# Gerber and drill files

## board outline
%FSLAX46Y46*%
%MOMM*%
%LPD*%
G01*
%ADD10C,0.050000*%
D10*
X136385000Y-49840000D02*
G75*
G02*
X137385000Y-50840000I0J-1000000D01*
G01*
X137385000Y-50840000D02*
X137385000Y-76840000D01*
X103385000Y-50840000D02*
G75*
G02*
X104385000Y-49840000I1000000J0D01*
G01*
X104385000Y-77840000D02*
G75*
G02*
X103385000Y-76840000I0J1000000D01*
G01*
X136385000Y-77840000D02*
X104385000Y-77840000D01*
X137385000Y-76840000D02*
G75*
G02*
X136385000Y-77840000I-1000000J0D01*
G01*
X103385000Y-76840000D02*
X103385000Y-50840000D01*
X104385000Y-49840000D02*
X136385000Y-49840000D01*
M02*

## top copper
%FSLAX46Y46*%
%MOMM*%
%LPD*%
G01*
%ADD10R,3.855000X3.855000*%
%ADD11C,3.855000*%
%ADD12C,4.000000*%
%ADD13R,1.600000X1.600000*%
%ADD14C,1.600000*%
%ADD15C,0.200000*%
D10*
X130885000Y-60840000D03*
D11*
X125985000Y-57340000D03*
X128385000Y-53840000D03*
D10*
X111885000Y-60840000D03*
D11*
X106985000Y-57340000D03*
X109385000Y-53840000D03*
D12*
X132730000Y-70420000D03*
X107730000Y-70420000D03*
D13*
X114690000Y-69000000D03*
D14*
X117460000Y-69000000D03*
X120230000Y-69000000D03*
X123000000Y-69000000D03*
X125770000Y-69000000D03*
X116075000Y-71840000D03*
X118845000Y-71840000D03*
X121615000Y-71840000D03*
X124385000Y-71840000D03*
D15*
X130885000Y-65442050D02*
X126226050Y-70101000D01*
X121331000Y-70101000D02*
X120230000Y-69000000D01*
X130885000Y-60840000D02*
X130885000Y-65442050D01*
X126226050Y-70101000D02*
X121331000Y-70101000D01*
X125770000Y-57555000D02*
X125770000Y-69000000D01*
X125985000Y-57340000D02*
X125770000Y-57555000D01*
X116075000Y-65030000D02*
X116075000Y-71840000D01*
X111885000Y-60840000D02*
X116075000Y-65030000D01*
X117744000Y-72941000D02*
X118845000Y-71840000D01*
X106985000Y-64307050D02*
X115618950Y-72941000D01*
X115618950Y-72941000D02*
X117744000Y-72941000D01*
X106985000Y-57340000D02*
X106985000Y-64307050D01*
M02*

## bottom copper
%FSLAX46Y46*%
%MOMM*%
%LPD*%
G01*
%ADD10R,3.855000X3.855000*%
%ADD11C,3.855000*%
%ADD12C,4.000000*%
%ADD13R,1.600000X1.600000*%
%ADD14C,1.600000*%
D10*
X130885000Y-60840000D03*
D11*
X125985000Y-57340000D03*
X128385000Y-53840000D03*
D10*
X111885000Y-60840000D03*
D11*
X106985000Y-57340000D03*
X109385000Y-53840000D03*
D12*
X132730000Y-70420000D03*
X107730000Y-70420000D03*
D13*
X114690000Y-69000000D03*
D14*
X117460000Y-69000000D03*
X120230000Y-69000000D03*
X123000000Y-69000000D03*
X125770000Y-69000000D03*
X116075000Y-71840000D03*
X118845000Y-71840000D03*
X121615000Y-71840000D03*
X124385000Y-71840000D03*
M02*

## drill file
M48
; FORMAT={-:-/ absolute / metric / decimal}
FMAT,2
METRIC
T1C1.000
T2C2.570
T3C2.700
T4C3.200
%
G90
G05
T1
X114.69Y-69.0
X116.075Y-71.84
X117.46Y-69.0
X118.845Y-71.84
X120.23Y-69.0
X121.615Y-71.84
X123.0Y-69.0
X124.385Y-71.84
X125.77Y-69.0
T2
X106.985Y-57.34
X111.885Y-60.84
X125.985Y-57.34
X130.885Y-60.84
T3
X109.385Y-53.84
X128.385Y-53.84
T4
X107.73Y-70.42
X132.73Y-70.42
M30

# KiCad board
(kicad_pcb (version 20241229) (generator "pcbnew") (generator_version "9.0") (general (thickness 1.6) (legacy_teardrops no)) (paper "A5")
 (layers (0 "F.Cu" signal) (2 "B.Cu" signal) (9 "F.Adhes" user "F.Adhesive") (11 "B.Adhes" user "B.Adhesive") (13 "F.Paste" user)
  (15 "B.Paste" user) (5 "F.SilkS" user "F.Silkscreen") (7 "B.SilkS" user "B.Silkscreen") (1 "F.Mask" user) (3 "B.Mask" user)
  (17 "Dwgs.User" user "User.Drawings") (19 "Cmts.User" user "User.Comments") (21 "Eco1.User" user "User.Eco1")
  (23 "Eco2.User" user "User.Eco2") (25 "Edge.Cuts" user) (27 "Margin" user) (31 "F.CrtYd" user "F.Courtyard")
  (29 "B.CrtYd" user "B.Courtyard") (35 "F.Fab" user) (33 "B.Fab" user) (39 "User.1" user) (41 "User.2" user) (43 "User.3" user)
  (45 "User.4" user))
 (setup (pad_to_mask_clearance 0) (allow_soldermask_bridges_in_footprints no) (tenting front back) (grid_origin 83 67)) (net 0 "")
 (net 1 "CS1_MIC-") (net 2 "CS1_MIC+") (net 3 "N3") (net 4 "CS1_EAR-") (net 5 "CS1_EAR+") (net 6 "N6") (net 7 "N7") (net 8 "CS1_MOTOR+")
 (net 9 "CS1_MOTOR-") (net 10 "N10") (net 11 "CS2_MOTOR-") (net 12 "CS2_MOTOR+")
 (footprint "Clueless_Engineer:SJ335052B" (layer "F.Cu") (at 130.885 60.84)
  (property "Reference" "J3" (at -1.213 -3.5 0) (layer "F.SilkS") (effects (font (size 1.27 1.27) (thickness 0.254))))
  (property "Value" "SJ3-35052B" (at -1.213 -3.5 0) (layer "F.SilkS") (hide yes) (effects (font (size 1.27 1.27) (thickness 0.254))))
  (pad "1" thru_hole rect (at 0 0) (size 3.855 3.855) (drill 2.57) (layers "*.Cu" "*.Mask") (remove_unused_layers no) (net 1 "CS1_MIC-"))
  (pad "2" thru_hole circle (at -4.9 -3.5) (size 3.855 3.855) (drill 2.57) (layers "*.Cu" "*.Mask") (remove_unused_layers no)
   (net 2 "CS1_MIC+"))
  (pad "4" thru_hole circle (at -2.5 -7) (size 3.855 3.855) (drill 2.7) (layers "*.Cu" "*.Mask") (remove_unused_layers no) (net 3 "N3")))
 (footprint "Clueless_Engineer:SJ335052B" (layer "F.Cu") (at 111.885 60.84)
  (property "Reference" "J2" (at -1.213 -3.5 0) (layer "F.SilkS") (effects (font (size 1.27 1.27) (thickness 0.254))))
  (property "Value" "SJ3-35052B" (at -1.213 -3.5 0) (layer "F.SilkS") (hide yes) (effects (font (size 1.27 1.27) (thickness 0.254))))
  (pad "1" thru_hole rect (at 0 0) (size 3.855 3.855) (drill 2.57) (layers "*.Cu" "*.Mask") (remove_unused_layers no) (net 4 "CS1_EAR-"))
  (pad "2" thru_hole circle (at -4.9 -3.5) (size 3.855 3.855) (drill 2.57) (layers "*.Cu" "*.Mask") (remove_unused_layers no)
   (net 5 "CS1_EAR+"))
  (pad "4" thru_hole circle (at -2.5 -7) (size 3.855 3.855) (drill 2.7) (layers "*.Cu" "*.Mask") (remove_unused_layers no) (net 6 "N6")))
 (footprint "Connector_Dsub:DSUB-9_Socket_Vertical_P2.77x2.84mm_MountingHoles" (layer "B.Cu") (at 114.69 69 180)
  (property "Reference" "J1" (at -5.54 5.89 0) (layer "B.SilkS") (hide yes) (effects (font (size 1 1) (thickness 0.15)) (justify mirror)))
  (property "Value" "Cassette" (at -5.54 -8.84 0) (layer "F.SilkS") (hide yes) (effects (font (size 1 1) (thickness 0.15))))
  (pad "0" thru_hole circle (at -18.04 -1.42 180) (size 4 4) (drill 3.2) (layers "*.Cu" "*.Mask") (remove_unused_layers no) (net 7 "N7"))
  (pad "0" thru_hole circle (at 6.96 -1.42 180) (size 4 4) (drill 3.2) (layers "*.Cu" "*.Mask") (remove_unused_layers no) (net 7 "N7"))
  (pad "1" thru_hole rect (at 0 0 180) (size 1.6 1.6) (drill 1) (layers "*.Cu" "*.Mask") (remove_unused_layers no) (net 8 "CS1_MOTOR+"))
  (pad "2" thru_hole circle (at -2.77 0 180) (size 1.6 1.6) (drill 1) (layers "*.Cu" "*.Mask") (remove_unused_layers no)
   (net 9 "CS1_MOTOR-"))
  (pad "3" thru_hole circle (at -5.54 0 180) (size 1.6 1.6) (drill 1) (layers "*.Cu" "*.Mask") (remove_unused_layers no) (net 1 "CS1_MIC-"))
  (pad "4" thru_hole circle (at -8.31 0 180) (size 1.6 1.6) (drill 1) (layers "*.Cu" "*.Mask") (remove_unused_layers no) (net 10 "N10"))
  (pad "5" thru_hole circle (at -11.08 0 180) (size 1.6 1.6) (drill 1) (layers "*.Cu" "*.Mask") (remove_unused_layers no) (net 2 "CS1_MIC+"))
  (pad "6" thru_hole circle (at -1.385 -2.84 180) (size 1.6 1.6) (drill 1) (layers "*.Cu" "*.Mask") (remove_unused_layers no)
   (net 4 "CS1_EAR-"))
  (pad "7" thru_hole circle (at -4.155 -2.84 180) (size 1.6 1.6) (drill 1) (layers "*.Cu" "*.Mask") (remove_unused_layers no)
   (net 5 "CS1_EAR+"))
  (pad "8" thru_hole circle (at -6.925 -2.84 180) (size 1.6 1.6) (drill 1) (layers "*.Cu" "*.Mask") (remove_unused_layers no)
   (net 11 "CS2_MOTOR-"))
  (pad "9" thru_hole circle (at -9.695 -2.84 180) (size 1.6 1.6) (drill 1) (layers "*.Cu" "*.Mask") (remove_unused_layers no)
   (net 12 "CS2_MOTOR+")))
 (gr_arc (start 136.385 49.84) (mid 137.092107 50.132893) (end 137.385 50.84) (stroke (width 0.05) (type default)) (layer "Edge.Cuts"))
 (gr_line (start 137.385 50.84) (end 137.385 76.84) (stroke (width 0.05) (type default)) (layer "Edge.Cuts"))
 (gr_arc (start 103.385 50.84) (mid 103.677893 50.132893) (end 104.385 49.84) (stroke (width 0.05) (type default)) (layer "Edge.Cuts"))
 (gr_arc (start 104.385 77.84) (mid 103.677893 77.547107) (end 103.385 76.84) (stroke (width 0.05) (type default)) (layer "Edge.Cuts"))
 (gr_line (start 136.385 77.84) (end 104.385 77.84) (stroke (width 0.05) (type default)) (layer "Edge.Cuts"))
 (gr_arc (start 137.385 76.84) (mid 137.092107 77.547107) (end 136.385 77.84) (stroke (width 0.05) (type default)) (layer "Edge.Cuts"))
 (gr_line (start 103.385 76.84) (end 103.385 50.84) (stroke (width 0.05) (type default)) (layer "Edge.Cuts"))
 (gr_line (start 104.385 49.84) (end 136.385 49.84) (stroke (width 0.05) (type default)) (layer "Edge.Cuts"))
 (segment (start 130.885 65.44205) (end 126.22605 70.101) (width 0.2) (layer "F.Cu") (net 1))
 (segment (start 121.331 70.101) (end 120.23 69) (width 0.2) (layer "F.Cu") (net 1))
 (segment (start 130.885 60.84) (end 130.885 65.44205) (width 0.2) (layer "F.Cu") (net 1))
 (segment (start 126.22605 70.101) (end 121.331 70.101) (width 0.2) (layer "F.Cu") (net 1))
 (segment (start 125.77 57.555) (end 125.77 69) (width 0.2) (layer "F.Cu") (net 2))
 (segment (start 125.985 57.34) (end 125.77 57.555) (width 0.2) (layer "F.Cu") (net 2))
 (segment (start 116.075 65.03) (end 116.075 71.84) (width 0.2) (layer "F.Cu") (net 4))
 (segment (start 111.885 60.84) (end 116.075 65.03) (width 0.2) (layer "F.Cu") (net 4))
 (segment (start 117.744 72.941) (end 118.845 71.84) (width 0.2) (layer "F.Cu") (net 5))
 (segment (start 106.985 64.30705) (end 115.61895 72.941) (width 0.2) (layer "F.Cu") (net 5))
 (segment (start 115.61895 72.941) (end 117.744 72.941) (width 0.2) (layer "F.Cu") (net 5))
 (segment (start 106.985 57.34) (end 106.985 64.30705) (width 0.2) (layer "F.Cu") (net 5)))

